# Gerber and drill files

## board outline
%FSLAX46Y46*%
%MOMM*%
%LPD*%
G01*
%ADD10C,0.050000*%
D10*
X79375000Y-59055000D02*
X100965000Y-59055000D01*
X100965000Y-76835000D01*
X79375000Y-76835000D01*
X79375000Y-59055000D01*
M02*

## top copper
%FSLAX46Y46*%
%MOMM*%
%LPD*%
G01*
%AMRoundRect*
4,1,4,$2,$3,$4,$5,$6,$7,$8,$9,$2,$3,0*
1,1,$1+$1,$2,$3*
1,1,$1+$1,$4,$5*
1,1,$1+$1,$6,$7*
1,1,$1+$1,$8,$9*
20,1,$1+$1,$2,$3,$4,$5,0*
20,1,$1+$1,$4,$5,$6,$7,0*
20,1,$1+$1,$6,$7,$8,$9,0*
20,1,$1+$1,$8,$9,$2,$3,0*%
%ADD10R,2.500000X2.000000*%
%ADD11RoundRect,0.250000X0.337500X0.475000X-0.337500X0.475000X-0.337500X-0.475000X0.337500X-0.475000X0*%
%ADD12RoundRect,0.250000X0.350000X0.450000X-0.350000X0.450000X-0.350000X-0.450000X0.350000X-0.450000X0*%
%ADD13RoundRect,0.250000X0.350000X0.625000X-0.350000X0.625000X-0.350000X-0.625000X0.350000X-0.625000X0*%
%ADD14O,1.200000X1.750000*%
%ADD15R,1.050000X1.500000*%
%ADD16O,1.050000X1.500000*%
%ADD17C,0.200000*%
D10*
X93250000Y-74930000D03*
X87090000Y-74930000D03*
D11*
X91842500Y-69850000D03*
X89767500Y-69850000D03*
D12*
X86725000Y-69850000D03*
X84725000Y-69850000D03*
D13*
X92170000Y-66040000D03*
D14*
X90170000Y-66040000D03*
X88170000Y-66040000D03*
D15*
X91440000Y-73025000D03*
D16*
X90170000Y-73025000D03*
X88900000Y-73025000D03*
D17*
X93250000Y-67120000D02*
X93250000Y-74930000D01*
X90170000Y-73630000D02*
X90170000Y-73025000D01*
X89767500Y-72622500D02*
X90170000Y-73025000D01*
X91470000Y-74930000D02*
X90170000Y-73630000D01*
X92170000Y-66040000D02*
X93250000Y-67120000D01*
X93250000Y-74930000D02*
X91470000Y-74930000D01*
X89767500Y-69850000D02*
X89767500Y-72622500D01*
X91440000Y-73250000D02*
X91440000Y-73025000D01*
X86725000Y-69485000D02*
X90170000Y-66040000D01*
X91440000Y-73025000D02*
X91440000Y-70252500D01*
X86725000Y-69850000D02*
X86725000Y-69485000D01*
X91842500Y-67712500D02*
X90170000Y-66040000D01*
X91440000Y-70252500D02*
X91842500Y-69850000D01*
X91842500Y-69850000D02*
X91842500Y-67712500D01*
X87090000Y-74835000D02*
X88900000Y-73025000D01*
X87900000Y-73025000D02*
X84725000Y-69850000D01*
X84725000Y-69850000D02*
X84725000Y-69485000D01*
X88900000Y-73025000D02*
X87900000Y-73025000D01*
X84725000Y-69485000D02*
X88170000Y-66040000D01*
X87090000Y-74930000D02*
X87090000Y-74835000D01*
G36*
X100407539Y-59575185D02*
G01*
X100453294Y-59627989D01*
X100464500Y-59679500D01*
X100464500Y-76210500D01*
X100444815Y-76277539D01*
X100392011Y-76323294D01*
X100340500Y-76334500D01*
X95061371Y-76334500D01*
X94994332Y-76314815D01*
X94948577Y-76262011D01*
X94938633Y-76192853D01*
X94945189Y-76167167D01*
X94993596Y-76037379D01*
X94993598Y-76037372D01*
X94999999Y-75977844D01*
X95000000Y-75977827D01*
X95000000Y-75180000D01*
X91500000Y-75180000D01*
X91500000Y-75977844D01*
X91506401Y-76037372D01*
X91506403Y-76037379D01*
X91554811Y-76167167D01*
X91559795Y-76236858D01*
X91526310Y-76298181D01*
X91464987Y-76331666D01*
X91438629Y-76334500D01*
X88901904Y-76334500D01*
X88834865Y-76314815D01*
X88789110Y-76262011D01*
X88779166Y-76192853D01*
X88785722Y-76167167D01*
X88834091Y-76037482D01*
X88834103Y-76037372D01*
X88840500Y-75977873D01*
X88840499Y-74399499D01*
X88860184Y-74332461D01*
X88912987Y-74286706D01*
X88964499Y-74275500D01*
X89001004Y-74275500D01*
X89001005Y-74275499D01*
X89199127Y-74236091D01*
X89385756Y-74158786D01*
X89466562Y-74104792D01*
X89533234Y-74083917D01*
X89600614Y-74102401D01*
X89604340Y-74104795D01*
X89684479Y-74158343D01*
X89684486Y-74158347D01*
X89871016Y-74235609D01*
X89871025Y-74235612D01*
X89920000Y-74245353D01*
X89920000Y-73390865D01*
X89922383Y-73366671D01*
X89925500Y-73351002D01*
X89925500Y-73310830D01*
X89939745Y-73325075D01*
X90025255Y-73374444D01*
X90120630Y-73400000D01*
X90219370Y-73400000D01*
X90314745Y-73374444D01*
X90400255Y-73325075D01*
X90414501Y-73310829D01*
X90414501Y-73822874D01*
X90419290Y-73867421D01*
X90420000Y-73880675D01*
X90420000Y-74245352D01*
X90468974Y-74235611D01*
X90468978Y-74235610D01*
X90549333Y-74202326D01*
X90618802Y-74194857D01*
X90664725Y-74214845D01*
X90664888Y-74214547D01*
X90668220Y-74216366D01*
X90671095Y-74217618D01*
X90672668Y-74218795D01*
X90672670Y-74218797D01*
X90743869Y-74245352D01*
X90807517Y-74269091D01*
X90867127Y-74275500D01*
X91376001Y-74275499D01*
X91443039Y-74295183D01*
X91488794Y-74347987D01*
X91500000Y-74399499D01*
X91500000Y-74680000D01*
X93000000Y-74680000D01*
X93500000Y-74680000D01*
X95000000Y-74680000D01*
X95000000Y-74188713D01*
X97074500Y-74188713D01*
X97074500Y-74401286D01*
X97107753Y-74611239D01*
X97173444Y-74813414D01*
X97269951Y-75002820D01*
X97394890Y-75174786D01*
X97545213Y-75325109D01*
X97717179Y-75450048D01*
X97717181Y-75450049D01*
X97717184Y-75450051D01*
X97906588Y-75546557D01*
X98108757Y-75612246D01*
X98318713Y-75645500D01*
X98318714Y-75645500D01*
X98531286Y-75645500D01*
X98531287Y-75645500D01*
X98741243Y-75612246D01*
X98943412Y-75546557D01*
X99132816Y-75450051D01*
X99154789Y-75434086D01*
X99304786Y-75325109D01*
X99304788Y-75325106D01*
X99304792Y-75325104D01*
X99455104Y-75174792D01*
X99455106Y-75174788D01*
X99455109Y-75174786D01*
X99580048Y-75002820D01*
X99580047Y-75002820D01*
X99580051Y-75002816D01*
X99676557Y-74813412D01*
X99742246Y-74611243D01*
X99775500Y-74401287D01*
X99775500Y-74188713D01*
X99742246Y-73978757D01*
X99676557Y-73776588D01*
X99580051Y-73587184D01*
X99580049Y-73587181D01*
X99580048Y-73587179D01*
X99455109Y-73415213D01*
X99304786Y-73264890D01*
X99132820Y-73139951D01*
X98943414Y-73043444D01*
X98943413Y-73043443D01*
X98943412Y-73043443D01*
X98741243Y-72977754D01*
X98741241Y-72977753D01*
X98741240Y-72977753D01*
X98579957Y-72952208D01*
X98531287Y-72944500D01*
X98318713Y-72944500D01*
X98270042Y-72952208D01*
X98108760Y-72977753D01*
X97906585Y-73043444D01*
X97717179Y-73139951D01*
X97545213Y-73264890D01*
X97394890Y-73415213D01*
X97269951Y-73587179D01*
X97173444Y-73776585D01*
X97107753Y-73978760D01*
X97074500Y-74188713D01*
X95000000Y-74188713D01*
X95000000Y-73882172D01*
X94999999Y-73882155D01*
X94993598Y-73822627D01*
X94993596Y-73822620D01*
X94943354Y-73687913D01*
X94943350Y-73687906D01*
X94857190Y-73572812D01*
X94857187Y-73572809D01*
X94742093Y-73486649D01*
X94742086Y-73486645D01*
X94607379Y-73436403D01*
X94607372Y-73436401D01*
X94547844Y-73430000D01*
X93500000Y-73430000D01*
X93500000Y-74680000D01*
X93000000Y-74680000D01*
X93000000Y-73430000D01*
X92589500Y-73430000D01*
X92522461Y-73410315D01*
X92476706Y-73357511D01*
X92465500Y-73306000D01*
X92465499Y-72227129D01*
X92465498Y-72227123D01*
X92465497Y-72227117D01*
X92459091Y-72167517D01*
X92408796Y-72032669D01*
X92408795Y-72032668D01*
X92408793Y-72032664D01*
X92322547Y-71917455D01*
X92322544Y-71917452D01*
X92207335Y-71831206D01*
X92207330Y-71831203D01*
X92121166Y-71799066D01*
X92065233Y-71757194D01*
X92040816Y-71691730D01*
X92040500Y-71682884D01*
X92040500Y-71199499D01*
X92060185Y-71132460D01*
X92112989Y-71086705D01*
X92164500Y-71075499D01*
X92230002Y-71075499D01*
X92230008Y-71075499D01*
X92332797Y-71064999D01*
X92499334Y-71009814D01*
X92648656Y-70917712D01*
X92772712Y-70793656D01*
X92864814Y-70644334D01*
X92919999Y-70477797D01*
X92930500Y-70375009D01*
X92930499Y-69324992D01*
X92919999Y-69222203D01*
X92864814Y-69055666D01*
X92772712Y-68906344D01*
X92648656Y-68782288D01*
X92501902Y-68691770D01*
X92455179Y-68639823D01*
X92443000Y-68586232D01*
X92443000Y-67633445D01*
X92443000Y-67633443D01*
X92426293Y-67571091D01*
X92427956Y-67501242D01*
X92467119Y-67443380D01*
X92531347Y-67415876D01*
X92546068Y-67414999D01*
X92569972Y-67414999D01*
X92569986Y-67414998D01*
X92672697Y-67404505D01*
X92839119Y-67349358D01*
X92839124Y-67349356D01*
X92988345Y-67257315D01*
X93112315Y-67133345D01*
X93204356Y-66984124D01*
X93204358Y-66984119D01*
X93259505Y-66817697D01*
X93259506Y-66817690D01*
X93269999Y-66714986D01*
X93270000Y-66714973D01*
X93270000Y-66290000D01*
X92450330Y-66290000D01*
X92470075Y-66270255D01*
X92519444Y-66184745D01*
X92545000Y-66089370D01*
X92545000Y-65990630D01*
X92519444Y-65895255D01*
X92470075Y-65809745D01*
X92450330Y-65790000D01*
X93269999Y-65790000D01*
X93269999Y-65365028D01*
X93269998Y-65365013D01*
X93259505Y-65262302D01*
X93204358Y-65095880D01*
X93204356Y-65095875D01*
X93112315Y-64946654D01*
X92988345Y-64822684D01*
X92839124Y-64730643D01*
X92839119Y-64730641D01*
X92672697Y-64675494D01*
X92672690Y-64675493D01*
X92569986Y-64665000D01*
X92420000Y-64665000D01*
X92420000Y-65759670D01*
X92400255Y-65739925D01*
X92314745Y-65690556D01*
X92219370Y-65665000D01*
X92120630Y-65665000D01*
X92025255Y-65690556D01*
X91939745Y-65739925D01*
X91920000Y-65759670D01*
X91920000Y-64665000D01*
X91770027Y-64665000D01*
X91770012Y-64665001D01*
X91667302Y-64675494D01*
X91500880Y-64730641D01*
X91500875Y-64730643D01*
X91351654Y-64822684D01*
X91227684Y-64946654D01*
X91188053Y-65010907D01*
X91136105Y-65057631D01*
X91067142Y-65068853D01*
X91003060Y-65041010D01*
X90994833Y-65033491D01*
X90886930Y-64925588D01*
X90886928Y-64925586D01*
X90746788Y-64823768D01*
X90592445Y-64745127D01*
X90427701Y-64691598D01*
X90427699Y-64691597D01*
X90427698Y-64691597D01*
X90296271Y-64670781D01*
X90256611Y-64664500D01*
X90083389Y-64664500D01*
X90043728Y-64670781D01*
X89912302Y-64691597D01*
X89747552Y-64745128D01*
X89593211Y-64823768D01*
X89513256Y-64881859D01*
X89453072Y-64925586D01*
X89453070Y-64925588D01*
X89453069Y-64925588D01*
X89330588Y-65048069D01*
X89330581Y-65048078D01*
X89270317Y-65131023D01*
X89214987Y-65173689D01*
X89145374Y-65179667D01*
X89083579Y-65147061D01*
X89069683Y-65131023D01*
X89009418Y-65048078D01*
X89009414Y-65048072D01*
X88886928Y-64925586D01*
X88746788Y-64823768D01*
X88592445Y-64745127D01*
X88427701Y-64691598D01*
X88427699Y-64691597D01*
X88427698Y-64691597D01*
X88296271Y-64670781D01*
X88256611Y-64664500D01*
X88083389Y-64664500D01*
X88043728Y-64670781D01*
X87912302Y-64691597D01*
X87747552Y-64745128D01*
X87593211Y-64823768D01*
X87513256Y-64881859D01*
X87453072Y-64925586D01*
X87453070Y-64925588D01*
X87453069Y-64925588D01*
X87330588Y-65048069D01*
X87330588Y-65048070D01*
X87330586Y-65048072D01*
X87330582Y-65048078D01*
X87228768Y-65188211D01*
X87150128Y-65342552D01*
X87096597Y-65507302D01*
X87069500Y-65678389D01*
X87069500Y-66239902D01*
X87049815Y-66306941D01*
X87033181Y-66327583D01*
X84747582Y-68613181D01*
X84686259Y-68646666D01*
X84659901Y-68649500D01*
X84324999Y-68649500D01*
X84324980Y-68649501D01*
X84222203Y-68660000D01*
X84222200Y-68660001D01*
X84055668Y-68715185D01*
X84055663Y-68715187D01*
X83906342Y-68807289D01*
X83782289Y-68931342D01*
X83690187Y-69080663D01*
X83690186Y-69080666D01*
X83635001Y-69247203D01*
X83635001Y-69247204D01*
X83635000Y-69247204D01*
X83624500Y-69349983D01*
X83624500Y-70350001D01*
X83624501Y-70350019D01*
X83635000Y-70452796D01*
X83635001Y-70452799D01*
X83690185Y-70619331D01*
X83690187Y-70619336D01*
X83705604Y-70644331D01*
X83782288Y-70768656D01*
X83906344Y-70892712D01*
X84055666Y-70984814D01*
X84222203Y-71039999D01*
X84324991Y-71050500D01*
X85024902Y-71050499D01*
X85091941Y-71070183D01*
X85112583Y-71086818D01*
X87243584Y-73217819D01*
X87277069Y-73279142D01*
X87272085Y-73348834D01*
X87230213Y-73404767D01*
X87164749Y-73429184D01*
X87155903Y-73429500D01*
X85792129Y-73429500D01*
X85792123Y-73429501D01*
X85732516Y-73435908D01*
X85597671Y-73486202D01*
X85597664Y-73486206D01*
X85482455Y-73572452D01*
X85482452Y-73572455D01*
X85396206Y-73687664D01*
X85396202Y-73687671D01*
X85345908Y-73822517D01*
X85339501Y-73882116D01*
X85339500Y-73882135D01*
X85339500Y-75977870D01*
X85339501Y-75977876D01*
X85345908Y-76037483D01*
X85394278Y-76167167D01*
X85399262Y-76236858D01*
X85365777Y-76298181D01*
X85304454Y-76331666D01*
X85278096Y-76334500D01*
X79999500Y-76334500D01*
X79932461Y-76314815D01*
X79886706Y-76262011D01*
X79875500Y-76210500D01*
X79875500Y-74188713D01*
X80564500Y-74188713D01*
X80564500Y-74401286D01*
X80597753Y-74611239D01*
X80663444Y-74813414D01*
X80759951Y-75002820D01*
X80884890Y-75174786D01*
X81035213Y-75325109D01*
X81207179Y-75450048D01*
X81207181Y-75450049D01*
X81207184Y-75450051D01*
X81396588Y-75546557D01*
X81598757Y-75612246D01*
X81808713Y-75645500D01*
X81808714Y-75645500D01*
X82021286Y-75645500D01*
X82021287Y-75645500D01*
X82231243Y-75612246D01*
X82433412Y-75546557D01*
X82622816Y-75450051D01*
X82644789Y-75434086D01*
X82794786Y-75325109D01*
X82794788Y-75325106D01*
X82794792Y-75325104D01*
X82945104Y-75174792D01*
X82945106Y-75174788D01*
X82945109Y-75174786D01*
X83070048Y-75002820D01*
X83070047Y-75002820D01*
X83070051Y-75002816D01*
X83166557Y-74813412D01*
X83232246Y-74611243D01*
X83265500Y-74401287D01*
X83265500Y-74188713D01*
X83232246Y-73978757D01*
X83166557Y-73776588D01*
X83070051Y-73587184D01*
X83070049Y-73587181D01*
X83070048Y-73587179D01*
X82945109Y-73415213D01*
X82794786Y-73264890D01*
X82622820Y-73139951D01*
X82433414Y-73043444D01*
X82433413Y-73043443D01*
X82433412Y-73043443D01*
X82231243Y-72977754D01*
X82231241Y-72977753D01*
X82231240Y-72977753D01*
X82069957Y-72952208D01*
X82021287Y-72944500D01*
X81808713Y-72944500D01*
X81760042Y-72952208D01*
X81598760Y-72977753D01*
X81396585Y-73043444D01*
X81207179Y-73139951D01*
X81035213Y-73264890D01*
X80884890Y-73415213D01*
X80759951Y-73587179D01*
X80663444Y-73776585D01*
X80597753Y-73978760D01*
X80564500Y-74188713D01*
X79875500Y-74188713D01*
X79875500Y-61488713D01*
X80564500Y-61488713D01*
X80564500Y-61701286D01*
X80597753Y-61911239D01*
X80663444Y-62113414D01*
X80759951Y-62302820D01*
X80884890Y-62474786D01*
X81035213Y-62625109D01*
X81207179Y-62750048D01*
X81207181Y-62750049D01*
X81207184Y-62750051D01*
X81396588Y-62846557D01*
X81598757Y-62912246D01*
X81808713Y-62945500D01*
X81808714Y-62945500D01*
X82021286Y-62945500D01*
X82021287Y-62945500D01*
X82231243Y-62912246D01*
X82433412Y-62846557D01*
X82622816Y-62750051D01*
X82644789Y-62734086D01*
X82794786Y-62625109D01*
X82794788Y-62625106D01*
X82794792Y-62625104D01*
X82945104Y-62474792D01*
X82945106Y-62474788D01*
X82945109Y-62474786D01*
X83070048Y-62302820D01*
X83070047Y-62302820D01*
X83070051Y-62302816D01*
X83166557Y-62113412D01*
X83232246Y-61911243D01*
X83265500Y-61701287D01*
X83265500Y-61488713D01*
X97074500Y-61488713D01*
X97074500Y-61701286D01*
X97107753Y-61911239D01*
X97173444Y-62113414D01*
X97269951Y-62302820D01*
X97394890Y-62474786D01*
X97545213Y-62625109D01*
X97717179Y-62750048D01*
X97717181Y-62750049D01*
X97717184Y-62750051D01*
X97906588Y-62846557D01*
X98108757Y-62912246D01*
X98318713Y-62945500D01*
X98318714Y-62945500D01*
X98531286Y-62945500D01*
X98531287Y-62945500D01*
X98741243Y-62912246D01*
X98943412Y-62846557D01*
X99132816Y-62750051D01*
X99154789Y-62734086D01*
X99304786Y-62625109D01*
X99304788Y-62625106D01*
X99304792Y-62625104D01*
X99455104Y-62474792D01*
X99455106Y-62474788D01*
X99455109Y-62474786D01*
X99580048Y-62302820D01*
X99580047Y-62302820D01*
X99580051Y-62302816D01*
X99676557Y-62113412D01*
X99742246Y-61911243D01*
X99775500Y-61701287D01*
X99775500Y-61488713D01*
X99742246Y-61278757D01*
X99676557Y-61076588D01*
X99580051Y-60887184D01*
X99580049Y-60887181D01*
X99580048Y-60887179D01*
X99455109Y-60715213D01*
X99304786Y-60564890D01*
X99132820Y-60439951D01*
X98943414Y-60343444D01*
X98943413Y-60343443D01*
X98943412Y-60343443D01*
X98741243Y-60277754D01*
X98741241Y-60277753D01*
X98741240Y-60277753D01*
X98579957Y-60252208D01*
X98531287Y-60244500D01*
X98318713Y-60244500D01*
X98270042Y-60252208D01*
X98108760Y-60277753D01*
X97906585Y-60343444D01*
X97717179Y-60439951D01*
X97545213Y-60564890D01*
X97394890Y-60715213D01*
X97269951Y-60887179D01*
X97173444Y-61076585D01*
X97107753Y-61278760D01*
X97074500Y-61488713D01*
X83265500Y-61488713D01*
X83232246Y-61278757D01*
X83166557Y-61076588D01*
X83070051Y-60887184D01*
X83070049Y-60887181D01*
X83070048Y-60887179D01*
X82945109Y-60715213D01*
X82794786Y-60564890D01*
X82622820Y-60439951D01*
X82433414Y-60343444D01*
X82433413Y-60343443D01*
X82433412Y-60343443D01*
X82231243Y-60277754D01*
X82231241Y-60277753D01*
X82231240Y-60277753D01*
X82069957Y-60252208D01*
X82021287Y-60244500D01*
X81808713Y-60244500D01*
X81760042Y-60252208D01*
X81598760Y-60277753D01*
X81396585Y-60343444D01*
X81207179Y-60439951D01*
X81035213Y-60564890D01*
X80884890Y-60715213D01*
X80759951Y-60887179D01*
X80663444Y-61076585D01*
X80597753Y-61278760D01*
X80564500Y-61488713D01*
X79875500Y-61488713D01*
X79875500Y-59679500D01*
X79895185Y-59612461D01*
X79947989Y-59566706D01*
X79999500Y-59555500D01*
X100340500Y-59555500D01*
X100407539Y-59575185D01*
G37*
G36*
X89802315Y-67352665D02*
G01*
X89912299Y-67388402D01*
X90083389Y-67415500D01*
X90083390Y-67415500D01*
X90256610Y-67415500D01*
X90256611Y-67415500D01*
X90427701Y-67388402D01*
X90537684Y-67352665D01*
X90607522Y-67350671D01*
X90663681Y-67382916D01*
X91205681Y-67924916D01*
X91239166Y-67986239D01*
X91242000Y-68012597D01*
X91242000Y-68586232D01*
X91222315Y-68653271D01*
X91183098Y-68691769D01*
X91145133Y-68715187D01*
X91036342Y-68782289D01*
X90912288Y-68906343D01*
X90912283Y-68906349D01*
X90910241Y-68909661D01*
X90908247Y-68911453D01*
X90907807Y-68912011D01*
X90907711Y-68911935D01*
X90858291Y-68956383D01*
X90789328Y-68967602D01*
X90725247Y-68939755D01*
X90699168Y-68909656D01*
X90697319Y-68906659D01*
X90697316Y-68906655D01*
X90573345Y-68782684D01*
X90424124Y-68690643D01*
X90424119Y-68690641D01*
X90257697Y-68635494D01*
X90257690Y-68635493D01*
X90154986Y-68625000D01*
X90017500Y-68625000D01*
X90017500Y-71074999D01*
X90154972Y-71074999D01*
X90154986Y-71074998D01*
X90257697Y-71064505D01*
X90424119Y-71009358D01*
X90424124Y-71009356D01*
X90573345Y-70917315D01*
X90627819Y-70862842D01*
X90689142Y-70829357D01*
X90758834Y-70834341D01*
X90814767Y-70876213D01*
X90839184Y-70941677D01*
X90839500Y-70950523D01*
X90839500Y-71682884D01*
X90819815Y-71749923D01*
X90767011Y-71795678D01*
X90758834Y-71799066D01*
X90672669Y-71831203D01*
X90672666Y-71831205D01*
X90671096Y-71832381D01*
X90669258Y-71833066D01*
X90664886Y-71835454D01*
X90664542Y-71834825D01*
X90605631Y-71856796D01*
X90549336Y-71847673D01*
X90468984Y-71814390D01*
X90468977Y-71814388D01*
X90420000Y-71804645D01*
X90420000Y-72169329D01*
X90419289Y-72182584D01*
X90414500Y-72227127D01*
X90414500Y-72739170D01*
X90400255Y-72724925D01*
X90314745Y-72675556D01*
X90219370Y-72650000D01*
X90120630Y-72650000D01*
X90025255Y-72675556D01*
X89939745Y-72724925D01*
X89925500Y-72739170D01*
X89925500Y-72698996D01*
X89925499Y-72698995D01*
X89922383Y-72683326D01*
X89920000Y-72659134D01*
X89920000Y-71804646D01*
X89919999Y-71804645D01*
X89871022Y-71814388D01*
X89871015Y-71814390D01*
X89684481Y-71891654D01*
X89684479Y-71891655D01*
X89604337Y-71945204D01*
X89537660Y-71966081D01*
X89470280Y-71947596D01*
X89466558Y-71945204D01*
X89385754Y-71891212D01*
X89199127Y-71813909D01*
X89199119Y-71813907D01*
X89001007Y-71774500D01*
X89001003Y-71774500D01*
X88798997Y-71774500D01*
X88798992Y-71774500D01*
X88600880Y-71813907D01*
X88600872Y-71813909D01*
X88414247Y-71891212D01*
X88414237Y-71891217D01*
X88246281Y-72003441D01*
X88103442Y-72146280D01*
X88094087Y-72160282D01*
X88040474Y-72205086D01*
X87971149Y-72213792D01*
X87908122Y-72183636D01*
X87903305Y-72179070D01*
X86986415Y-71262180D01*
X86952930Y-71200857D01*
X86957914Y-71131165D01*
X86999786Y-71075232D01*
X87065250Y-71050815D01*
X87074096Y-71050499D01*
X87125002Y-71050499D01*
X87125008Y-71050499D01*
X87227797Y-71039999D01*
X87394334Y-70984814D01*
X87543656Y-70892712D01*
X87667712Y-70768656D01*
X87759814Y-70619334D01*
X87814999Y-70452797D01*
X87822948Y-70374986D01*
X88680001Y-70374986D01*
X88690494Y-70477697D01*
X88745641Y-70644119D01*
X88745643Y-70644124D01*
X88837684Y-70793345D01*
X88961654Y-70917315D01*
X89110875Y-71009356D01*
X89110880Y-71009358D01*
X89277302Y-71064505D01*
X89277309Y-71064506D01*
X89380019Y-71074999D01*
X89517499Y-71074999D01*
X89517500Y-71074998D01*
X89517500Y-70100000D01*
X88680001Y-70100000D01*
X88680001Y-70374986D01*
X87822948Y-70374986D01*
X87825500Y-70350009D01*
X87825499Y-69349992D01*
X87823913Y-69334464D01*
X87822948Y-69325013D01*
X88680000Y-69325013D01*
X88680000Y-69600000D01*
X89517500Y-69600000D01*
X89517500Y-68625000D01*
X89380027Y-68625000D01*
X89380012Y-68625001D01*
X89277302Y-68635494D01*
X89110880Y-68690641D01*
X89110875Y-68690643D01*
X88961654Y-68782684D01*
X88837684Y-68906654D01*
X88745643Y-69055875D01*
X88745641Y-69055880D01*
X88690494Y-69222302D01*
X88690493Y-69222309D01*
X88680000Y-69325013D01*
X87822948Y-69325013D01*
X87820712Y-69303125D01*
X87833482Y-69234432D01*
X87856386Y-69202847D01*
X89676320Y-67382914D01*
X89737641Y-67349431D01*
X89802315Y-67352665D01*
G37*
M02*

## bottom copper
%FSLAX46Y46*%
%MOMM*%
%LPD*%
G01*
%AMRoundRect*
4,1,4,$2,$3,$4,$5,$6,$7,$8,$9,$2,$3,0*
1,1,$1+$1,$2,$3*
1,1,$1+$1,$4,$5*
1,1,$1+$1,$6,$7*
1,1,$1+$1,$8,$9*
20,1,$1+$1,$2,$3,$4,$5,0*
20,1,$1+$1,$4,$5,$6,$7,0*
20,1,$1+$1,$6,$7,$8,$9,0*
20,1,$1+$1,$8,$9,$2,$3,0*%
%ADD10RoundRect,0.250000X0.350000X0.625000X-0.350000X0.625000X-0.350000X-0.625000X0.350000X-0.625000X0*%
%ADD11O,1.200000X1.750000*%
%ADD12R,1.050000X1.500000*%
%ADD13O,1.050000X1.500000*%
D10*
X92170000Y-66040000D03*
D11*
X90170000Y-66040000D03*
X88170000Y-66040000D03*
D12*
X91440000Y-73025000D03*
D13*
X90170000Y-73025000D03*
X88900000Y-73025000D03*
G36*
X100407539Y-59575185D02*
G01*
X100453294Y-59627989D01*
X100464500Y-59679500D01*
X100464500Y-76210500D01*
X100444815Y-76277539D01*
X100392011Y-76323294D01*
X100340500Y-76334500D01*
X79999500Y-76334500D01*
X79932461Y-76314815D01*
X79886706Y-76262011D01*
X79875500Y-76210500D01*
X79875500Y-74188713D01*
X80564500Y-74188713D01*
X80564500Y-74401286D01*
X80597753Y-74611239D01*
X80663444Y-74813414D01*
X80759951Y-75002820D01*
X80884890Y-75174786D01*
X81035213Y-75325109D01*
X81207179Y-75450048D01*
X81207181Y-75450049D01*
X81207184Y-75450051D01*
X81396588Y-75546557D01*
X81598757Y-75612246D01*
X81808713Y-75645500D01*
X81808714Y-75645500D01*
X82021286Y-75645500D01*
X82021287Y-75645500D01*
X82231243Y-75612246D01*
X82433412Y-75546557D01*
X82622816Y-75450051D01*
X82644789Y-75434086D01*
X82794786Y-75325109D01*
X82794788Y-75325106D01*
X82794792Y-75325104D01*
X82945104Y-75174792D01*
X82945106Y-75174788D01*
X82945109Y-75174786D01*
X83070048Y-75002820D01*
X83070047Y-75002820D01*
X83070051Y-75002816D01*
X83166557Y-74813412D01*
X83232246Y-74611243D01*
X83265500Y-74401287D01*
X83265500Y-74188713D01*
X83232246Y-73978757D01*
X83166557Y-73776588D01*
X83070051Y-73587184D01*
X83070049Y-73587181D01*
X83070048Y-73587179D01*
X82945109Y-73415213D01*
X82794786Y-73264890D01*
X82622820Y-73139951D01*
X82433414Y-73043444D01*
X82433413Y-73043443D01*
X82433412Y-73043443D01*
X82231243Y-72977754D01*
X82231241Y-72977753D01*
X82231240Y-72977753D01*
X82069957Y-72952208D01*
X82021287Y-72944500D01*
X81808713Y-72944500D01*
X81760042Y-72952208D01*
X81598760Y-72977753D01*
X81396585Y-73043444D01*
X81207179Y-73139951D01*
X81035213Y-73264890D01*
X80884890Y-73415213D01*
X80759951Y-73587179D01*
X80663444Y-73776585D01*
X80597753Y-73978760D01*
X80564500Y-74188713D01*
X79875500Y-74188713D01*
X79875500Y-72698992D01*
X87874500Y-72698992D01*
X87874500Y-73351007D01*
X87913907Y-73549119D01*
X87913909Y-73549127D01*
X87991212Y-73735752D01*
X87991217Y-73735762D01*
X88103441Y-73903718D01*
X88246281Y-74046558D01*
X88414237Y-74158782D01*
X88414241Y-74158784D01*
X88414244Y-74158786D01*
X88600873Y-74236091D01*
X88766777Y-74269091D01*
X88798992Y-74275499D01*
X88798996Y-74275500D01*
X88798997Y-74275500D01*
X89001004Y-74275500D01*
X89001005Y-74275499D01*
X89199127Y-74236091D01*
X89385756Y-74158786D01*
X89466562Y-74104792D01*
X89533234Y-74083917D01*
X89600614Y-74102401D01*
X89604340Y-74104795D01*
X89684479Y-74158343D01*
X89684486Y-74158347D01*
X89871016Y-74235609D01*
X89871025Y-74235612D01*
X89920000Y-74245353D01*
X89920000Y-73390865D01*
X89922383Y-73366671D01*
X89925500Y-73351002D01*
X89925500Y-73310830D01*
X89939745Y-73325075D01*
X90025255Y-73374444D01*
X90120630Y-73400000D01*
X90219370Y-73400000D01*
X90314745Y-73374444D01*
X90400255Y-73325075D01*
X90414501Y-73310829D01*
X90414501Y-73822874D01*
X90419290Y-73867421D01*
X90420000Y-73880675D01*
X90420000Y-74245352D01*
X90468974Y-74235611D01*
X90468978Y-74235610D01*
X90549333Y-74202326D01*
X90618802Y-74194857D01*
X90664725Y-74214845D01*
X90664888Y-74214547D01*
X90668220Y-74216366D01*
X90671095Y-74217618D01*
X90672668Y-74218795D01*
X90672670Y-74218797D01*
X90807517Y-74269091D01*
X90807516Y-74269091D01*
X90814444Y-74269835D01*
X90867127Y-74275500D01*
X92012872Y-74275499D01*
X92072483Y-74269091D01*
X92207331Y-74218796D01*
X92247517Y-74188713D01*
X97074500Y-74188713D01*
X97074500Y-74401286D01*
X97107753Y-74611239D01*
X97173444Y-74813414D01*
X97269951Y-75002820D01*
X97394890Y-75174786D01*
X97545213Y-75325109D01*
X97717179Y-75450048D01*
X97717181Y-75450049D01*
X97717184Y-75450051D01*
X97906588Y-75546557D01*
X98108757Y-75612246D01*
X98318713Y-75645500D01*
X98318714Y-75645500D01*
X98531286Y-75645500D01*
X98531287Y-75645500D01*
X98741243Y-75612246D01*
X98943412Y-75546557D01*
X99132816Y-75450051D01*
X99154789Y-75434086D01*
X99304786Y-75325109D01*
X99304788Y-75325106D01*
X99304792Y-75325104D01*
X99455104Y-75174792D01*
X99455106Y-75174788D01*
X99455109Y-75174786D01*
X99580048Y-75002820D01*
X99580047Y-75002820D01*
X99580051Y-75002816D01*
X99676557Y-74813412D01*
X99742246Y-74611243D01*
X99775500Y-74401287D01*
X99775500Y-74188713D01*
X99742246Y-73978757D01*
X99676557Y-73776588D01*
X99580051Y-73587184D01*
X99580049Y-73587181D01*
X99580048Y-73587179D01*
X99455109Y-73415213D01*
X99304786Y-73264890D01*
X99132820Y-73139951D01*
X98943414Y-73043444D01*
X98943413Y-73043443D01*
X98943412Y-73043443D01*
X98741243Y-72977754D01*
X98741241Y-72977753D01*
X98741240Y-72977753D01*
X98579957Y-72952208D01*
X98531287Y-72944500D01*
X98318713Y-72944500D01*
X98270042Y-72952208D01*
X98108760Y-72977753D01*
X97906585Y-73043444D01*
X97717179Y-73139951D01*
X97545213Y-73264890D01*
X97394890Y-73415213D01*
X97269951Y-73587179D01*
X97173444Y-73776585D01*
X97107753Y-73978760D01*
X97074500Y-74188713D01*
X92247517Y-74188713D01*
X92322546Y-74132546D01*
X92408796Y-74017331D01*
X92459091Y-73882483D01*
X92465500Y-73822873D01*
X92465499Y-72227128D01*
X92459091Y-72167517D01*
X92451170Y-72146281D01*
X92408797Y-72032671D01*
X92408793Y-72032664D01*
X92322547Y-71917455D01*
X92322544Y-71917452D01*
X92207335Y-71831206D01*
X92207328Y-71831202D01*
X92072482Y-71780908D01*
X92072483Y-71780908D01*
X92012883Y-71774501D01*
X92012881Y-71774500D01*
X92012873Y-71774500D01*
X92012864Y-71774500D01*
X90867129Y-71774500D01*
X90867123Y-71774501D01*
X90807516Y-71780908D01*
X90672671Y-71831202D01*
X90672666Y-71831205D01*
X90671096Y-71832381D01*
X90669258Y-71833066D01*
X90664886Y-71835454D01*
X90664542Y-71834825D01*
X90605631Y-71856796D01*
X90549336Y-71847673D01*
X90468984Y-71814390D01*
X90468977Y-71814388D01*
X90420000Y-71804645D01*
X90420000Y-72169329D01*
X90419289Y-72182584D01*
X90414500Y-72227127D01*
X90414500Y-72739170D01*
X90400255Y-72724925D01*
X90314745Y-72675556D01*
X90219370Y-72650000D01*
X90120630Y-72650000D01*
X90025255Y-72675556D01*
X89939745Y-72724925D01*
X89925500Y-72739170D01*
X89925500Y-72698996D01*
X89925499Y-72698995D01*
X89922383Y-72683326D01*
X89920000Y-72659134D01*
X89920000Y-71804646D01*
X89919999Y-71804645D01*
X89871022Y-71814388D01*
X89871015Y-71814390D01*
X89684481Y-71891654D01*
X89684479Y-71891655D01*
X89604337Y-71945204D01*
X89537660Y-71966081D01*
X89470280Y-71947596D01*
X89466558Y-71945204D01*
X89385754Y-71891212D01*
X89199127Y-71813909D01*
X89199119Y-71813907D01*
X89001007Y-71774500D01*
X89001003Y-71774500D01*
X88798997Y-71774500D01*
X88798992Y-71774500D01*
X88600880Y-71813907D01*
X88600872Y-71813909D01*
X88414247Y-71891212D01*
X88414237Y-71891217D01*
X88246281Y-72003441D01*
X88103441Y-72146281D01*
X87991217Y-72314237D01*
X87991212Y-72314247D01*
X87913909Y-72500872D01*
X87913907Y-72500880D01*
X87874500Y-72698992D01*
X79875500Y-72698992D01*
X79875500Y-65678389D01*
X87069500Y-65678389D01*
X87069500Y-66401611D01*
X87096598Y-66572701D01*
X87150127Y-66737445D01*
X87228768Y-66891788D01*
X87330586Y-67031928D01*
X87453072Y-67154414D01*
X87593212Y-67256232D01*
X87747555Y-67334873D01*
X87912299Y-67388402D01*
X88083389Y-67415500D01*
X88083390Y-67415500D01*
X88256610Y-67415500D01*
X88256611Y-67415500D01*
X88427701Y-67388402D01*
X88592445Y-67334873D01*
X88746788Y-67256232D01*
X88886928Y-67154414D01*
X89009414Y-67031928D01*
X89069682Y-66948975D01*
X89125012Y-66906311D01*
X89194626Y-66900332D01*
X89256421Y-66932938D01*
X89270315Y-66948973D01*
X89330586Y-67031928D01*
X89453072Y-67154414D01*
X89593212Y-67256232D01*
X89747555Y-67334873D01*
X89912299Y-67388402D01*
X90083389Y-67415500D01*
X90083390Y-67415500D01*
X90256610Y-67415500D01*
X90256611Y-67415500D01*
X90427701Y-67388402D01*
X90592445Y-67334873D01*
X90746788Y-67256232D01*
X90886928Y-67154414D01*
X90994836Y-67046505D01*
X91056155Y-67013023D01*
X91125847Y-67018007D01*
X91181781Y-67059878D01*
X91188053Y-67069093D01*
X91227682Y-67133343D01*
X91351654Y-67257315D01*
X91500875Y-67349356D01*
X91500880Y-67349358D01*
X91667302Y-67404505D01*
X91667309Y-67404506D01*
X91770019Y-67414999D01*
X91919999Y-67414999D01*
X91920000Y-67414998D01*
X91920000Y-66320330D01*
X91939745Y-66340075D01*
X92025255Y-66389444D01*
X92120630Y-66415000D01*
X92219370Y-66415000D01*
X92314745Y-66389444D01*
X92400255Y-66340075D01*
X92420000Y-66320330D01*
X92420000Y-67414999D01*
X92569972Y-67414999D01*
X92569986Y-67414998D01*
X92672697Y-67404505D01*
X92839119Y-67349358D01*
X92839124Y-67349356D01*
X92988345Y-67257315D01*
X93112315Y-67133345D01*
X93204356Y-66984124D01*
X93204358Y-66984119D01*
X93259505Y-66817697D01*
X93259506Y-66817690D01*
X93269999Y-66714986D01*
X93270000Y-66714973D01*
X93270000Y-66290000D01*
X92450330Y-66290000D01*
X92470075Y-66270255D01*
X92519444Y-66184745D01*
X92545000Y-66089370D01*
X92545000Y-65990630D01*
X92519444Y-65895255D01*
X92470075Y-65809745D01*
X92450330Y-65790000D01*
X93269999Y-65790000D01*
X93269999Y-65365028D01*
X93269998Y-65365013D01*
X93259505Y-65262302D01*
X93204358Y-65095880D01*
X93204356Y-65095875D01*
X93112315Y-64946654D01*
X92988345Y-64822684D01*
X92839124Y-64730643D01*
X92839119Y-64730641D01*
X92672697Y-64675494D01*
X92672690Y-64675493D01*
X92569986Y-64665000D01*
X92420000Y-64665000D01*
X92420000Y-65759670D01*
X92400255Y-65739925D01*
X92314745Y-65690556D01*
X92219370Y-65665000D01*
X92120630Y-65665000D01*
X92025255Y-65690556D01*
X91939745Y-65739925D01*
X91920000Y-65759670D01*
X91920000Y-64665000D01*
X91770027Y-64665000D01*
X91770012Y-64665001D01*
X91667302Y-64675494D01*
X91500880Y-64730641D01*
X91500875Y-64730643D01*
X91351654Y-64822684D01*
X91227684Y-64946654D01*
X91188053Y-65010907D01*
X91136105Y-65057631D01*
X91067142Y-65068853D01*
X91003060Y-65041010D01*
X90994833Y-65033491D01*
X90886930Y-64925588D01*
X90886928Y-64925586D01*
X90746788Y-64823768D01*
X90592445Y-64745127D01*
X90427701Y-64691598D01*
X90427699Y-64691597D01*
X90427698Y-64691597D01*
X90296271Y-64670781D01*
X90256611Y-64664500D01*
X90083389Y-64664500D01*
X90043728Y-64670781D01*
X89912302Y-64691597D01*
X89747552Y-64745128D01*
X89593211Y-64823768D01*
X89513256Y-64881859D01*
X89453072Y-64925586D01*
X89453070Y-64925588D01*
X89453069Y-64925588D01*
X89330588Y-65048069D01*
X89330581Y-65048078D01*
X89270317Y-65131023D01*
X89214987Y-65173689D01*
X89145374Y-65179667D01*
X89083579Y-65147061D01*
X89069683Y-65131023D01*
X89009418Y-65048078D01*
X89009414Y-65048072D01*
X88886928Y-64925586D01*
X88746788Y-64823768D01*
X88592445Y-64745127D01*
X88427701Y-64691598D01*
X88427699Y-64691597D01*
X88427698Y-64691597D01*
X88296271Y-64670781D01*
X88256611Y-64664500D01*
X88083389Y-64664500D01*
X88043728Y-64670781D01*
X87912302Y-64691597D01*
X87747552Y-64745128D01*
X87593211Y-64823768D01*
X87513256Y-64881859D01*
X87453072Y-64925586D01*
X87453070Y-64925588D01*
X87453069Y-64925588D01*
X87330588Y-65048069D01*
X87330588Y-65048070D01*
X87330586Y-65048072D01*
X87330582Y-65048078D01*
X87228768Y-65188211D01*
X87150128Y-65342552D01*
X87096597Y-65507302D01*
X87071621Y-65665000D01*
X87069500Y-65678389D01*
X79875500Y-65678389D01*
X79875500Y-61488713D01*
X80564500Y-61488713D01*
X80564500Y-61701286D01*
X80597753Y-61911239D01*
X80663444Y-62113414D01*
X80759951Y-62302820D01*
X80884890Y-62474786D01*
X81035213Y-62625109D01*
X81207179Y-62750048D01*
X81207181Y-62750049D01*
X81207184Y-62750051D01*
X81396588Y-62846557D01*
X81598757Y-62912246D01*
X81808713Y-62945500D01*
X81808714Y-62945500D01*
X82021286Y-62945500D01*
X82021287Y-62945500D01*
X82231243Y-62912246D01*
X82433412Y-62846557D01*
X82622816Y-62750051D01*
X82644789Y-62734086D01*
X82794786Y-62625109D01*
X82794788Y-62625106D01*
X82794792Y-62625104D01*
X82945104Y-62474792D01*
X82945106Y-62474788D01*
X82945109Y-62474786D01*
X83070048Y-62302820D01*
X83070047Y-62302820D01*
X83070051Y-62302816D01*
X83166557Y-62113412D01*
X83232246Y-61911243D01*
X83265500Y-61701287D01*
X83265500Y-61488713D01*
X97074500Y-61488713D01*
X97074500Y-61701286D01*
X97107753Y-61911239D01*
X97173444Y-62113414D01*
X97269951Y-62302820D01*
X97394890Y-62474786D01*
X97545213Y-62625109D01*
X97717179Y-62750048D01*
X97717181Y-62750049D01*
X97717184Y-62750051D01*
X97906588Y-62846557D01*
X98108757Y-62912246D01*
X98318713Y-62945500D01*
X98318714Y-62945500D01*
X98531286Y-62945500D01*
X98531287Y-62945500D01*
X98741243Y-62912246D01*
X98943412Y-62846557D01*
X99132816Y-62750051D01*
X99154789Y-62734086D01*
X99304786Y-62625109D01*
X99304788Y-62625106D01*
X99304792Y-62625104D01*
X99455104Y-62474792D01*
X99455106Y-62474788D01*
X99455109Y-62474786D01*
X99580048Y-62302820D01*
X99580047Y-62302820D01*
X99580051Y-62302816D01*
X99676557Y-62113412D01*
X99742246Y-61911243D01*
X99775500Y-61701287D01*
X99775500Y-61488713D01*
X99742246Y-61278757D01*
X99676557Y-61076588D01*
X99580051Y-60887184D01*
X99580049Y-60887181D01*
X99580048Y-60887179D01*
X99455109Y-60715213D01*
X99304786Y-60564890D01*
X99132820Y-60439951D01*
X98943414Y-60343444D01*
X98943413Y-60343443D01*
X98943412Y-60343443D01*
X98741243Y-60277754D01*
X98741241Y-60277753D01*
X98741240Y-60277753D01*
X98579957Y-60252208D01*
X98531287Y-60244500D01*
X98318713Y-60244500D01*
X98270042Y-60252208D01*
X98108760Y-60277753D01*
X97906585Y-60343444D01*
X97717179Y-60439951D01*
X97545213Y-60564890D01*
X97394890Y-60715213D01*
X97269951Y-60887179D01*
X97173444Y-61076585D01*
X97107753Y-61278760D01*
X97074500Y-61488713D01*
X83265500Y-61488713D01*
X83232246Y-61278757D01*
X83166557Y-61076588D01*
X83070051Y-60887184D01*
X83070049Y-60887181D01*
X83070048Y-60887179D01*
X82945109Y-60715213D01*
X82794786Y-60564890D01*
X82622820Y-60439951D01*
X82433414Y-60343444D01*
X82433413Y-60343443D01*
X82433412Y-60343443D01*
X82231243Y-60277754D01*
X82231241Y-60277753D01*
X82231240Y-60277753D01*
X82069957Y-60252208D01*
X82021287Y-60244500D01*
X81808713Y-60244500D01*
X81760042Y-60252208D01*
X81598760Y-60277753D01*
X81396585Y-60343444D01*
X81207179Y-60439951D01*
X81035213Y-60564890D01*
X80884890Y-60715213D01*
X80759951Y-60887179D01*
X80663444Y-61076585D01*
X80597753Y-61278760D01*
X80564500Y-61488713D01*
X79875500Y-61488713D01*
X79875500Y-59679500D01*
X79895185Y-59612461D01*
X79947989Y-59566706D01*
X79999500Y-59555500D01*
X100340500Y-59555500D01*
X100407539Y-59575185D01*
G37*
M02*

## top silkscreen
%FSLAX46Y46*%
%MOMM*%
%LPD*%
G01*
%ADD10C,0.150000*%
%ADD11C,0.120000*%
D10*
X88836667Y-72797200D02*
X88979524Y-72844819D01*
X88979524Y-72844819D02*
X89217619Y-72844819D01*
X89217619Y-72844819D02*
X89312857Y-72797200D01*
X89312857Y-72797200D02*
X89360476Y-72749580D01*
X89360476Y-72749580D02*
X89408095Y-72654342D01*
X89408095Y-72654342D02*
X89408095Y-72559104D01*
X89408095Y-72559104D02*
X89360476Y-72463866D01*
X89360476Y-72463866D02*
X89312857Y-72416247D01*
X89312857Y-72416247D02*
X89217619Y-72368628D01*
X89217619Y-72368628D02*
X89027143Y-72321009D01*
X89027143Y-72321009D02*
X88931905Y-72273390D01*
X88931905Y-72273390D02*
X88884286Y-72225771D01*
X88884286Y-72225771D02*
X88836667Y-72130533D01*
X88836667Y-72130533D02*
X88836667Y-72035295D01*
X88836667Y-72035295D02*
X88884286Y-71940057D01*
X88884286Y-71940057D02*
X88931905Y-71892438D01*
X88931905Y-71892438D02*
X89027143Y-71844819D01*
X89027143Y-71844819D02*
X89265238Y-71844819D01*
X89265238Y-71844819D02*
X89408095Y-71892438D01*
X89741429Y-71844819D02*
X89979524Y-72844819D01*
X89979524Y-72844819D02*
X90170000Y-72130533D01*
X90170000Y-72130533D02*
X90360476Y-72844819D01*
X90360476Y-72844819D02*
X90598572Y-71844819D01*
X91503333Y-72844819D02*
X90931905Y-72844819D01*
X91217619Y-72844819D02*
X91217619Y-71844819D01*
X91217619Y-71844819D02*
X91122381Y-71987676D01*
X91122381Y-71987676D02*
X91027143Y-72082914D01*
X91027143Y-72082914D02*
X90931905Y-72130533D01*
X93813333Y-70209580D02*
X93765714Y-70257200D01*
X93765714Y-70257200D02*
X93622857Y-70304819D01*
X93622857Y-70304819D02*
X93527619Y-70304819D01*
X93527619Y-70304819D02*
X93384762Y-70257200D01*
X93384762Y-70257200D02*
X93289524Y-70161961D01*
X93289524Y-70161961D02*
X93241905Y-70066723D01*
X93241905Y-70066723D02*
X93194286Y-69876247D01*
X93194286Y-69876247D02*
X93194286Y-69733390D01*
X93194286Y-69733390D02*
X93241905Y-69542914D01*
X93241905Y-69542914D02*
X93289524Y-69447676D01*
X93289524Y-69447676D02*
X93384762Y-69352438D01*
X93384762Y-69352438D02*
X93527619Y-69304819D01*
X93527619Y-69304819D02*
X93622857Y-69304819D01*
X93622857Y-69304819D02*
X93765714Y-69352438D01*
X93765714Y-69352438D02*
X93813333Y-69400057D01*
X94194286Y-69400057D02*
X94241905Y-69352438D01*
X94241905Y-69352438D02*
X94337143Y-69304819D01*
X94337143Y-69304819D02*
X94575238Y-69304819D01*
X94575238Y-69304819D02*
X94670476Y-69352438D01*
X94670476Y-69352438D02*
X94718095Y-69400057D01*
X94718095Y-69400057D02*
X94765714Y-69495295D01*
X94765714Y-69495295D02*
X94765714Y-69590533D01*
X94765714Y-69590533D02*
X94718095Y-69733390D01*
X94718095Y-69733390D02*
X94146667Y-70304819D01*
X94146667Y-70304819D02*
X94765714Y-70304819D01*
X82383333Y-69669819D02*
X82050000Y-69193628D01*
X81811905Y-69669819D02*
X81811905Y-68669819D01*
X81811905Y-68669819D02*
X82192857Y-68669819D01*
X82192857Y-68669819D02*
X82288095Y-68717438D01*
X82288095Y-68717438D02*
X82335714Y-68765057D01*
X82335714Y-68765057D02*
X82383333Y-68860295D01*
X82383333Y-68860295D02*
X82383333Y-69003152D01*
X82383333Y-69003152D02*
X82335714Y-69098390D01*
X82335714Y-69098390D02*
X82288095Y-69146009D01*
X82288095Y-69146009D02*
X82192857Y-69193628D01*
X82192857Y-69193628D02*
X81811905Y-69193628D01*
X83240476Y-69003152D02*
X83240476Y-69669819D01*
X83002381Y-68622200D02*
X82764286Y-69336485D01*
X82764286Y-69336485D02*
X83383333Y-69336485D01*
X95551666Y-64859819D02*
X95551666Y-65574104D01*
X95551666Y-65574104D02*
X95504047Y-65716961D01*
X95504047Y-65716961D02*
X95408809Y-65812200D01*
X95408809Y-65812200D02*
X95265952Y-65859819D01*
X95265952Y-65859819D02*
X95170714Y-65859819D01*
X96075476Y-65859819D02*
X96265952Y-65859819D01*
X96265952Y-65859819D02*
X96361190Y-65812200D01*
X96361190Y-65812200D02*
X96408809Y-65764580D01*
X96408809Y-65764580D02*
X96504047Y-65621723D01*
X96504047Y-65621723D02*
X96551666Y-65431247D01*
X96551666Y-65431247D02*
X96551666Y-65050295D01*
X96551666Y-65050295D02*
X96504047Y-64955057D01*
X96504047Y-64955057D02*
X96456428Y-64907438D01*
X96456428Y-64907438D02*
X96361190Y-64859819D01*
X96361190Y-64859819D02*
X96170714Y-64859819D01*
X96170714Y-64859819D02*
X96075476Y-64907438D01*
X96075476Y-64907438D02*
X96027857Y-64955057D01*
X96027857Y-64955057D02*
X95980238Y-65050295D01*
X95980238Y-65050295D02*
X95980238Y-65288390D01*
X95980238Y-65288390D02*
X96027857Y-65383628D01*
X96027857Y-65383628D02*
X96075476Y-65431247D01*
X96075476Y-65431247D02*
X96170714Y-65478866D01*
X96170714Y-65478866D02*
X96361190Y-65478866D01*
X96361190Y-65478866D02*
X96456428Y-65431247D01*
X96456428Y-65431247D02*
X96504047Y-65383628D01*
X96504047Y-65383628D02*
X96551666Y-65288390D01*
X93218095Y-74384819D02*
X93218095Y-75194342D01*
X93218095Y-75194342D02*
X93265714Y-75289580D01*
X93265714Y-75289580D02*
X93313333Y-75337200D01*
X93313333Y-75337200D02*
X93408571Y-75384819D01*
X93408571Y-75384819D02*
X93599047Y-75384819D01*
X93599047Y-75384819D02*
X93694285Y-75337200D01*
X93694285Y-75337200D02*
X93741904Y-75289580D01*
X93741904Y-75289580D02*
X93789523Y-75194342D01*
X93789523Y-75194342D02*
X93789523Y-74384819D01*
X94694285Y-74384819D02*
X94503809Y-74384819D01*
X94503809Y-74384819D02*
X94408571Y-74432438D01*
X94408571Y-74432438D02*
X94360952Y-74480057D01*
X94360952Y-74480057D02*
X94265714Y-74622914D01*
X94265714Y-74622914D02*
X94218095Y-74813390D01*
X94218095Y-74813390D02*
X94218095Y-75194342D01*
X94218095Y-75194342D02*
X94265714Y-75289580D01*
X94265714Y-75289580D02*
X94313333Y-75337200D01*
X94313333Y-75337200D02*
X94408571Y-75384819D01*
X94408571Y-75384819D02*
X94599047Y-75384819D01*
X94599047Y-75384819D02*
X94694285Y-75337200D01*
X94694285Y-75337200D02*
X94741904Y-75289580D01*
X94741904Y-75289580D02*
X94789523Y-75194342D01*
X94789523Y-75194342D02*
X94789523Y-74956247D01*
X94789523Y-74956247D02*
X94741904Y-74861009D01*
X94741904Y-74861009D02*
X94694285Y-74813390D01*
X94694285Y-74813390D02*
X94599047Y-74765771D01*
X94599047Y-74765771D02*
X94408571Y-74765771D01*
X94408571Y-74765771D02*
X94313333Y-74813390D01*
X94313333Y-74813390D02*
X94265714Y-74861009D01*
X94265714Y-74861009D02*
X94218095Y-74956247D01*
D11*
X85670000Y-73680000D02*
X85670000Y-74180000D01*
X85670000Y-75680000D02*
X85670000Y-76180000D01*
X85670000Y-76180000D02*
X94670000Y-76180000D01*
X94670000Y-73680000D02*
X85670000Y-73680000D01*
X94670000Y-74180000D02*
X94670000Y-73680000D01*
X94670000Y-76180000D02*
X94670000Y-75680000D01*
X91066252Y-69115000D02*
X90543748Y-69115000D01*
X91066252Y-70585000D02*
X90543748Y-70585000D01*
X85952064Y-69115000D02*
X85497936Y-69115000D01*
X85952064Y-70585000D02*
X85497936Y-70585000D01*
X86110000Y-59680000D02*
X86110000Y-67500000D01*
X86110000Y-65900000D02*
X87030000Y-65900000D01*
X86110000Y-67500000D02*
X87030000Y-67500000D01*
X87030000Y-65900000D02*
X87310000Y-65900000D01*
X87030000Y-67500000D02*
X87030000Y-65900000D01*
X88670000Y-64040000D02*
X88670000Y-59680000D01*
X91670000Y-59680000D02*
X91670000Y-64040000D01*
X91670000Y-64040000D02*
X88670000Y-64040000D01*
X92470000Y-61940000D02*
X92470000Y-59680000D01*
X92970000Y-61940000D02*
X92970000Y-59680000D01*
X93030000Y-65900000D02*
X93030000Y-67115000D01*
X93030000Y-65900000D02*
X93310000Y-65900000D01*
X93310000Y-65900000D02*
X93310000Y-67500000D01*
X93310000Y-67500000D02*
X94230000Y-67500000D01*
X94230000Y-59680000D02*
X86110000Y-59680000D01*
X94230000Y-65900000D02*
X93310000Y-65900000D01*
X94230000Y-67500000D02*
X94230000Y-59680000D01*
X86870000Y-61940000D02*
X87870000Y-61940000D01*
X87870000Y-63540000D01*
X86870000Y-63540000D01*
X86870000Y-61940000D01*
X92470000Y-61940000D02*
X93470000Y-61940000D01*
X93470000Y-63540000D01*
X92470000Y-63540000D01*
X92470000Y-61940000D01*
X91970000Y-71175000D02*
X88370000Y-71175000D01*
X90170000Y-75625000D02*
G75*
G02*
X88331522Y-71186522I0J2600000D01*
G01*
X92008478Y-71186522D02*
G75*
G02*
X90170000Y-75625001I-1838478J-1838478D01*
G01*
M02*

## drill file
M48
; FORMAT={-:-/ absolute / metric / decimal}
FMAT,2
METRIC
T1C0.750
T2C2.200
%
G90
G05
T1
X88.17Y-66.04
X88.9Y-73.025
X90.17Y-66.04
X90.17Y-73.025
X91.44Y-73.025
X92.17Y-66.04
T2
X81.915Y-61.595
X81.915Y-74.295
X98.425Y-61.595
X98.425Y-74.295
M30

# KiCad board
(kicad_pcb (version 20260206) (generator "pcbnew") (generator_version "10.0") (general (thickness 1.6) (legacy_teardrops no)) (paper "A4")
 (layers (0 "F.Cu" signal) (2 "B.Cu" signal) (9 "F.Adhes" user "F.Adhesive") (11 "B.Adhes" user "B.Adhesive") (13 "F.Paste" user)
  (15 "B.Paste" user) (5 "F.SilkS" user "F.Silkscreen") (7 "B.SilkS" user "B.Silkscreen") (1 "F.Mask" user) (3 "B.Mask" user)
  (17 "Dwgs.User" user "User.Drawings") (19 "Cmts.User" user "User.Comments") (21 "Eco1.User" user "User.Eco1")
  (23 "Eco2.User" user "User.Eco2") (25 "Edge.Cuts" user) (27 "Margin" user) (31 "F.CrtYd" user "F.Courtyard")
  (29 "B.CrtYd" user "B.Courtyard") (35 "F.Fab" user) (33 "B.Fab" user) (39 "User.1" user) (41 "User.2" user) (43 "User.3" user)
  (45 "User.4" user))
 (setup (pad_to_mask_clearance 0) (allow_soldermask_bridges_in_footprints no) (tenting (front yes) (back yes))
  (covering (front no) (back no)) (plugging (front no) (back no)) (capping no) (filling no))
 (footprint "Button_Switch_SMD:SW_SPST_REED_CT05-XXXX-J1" (layer "F.Cu") (at 90.17 74.93 180)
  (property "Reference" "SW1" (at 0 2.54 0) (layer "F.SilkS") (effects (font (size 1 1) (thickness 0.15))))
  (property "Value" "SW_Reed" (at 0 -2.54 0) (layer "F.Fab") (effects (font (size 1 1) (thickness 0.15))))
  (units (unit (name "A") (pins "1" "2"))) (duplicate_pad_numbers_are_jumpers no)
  (fp_line (start 4.5 1.25) (end 4.5 0.75) (stroke (width 0.12) (type solid)) (layer "F.SilkS"))
  (fp_line (start 4.5 -0.75) (end 4.5 -1.25) (stroke (width 0.12) (type solid)) (layer "F.SilkS"))
  (fp_line (start 4.5 -1.25) (end -4.5 -1.25) (stroke (width 0.12) (type solid)) (layer "F.SilkS"))
  (fp_line (start -4.5 1.25) (end 4.5 1.25) (stroke (width 0.12) (type solid)) (layer "F.SilkS"))
  (fp_line (start -4.5 0.75) (end -4.5 1.25) (stroke (width 0.12) (type solid)) (layer "F.SilkS"))
  (fp_line (start -4.5 -1.25) (end -4.5 -0.75) (stroke (width 0.12) (type solid)) (layer "F.SilkS"))
  (pad "1" smd rect (at -3.08 0 180) (size 2.5 2) (layers "F.Cu" "F.Mask" "F.Paste") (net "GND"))
  (pad "2" smd rect (at 3.08 0 180) (size 2.5 2) (layers "F.Cu" "F.Mask" "F.Paste") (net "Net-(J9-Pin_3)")))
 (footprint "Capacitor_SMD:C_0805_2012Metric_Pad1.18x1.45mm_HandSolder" (layer "F.Cu") (at 90.805 69.85 180)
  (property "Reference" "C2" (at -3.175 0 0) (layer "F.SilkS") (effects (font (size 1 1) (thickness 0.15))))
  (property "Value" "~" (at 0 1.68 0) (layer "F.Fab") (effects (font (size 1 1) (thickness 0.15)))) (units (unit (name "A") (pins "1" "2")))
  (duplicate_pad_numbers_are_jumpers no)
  (fp_line (start -0.261252 0.735) (end 0.261252 0.735) (stroke (width 0.12) (type solid)) (layer "F.SilkS"))
  (fp_line (start -0.261252 -0.735) (end 0.261252 -0.735) (stroke (width 0.12) (type solid)) (layer "F.SilkS"))
  (pad "1" smd roundrect (at -1.0375 0 180) (size 1.175 1.45) (layers "F.Cu" "F.Mask" "F.Paste") (roundrect_rratio 0.212766) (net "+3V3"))
  (pad "2" smd roundrect (at 1.0375 0 180) (size 1.175 1.45) (layers "F.Cu" "F.Mask" "F.Paste") (roundrect_rratio 0.212766) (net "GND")))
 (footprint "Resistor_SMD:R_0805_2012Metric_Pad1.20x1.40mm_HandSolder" (layer "F.Cu") (at 85.725 69.85 180)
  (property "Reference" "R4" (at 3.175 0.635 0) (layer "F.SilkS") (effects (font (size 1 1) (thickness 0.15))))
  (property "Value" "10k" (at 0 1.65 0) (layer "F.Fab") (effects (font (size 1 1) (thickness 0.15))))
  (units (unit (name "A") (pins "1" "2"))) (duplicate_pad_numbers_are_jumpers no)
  (fp_line (start -0.227064 0.735) (end 0.227064 0.735) (stroke (width 0.12) (type solid)) (layer "F.SilkS"))
  (fp_line (start -0.227064 -0.735) (end 0.227064 -0.735) (stroke (width 0.12) (type solid)) (layer "F.SilkS"))
  (pad "1" smd roundrect (at -1 0 180) (size 1.2 1.4) (layers "F.Cu" "F.Mask" "F.Paste") (roundrect_rratio 0.208333) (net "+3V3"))
  (pad "2" smd roundrect (at 1 0 180) (size 1.2 1.4) (layers "F.Cu" "F.Mask" "F.Paste") (roundrect_rratio 0.208333) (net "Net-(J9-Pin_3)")))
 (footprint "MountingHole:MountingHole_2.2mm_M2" (layer "F.Cu") (at 98.425 61.595)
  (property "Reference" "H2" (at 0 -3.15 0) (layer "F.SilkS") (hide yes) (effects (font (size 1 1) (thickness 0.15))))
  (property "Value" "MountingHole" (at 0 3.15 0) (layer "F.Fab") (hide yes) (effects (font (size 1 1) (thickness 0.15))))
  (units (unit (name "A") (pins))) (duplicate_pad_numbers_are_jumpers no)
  (pad "" np_thru_hole circle (at 0 0) (size 2.2 2.2) (drill 2.2) (layers "*.Cu" "*.Mask")))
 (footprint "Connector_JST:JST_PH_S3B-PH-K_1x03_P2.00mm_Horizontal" (layer "F.Cu") (at 92.17 66.04 180)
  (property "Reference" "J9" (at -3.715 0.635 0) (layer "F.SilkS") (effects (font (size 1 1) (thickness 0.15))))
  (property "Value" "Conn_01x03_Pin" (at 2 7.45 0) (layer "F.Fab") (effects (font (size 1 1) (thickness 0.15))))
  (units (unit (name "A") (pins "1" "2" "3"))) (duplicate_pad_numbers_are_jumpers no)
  (fp_line (start 6.06 6.36) (end 6.06 -1.46) (stroke (width 0.12) (type solid)) (layer "F.SilkS"))
  (fp_line (start 6.06 0.14) (end 5.14 0.14) (stroke (width 0.12) (type solid)) (layer "F.SilkS"))
  (fp_line (start 6.06 -1.46) (end 5.14 -1.46) (stroke (width 0.12) (type solid)) (layer "F.SilkS"))
  (fp_line (start 5.14 0.14) (end 4.86 0.14) (stroke (width 0.12) (type solid)) (layer "F.SilkS"))
  (fp_line (start 5.14 -1.46) (end 5.14 0.14) (stroke (width 0.12) (type solid)) (layer "F.SilkS"))
  (fp_line (start 3.5 2) (end 3.5 6.36) (stroke (width 0.12) (type solid)) (layer "F.SilkS"))
  (fp_line (start 0.5 6.36) (end 0.5 2) (stroke (width 0.12) (type solid)) (layer "F.SilkS"))
  (fp_line (start 0.5 2) (end 3.5 2) (stroke (width 0.12) (type solid)) (layer "F.SilkS"))
  (fp_line (start -0.3 4.1) (end -0.3 6.36) (stroke (width 0.12) (type solid)) (layer "F.SilkS"))
  (fp_line (start -0.8 4.1) (end -0.8 6.36) (stroke (width 0.12) (type solid)) (layer "F.SilkS"))
  (fp_line (start -0.86 0.14) (end -0.86 -1.075) (stroke (width 0.12) (type solid)) (layer "F.SilkS"))
  (fp_line (start -0.86 0.14) (end -1.14 0.14) (stroke (width 0.12) (type solid)) (layer "F.SilkS"))
  (fp_line (start -1.14 0.14) (end -1.14 -1.46) (stroke (width 0.12) (type solid)) (layer "F.SilkS"))
  (fp_line (start -1.14 -1.46) (end -2.06 -1.46) (stroke (width 0.12) (type solid)) (layer "F.SilkS"))
  (fp_line (start -2.06 6.36) (end 6.06 6.36) (stroke (width 0.12) (type solid)) (layer "F.SilkS"))
  (fp_line (start -2.06 0.14) (end -1.14 0.14) (stroke (width 0.12) (type solid)) (layer "F.SilkS"))
  (fp_line (start -2.06 -1.46) (end -2.06 6.36) (stroke (width 0.12) (type solid)) (layer "F.SilkS"))
  (fp_rect (start 4.3 2.5) (end 5.3 4.1) (stroke (width 0.12) (type solid)) (fill no) (layer "F.SilkS"))
  (fp_rect (start -1.3 2.5) (end -0.3 4.1) (stroke (width 0.12) (type solid)) (fill no) (layer "F.SilkS"))
  (pad "1" thru_hole roundrect (at 0 0 180) (size 1.2 1.75) (drill 0.75) (layers "*.Cu" "*.Mask") (remove_unused_layers no)
   (roundrect_rratio 0.208333) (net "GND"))
  (pad "2" thru_hole oval (at 2 0 180) (size 1.2 1.75) (drill 0.75) (layers "*.Cu" "*.Mask") (remove_unused_layers no) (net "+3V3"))
  (pad "3" thru_hole oval (at 4 0 180) (size 1.2 1.75) (drill 0.75) (layers "*.Cu" "*.Mask") (remove_unused_layers no)
   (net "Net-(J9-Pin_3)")))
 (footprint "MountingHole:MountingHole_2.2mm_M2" (layer "F.Cu") (at 81.915 74.295)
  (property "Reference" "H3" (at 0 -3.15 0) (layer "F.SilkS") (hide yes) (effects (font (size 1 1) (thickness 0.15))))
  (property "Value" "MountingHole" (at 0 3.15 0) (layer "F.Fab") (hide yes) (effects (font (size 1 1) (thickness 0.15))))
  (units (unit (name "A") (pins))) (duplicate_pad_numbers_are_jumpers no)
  (pad "" np_thru_hole circle (at 0 0) (size 2.2 2.2) (drill 2.2) (layers "*.Cu" "*.Mask")))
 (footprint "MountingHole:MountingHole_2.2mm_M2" (layer "F.Cu") (at 98.425 74.295)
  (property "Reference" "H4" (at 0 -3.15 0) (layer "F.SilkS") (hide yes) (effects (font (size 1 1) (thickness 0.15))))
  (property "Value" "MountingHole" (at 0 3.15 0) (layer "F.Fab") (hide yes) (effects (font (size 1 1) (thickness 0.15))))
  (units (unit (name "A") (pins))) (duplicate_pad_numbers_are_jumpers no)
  (pad "" np_thru_hole circle (at 0 0) (size 2.2 2.2) (drill 2.2) (layers "*.Cu" "*.Mask")))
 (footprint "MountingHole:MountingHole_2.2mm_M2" (layer "F.Cu") (at 81.915 61.595)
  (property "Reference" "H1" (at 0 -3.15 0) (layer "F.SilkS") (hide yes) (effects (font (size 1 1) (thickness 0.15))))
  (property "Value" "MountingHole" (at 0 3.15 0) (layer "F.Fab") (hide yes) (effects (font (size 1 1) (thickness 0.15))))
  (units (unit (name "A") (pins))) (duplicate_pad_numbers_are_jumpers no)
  (pad "" np_thru_hole circle (at 0 0) (size 2.2 2.2) (drill 2.2) (layers "*.Cu" "*.Mask")))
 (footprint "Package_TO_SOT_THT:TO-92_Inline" (layer "F.Cu") (at 91.44 73.025 180)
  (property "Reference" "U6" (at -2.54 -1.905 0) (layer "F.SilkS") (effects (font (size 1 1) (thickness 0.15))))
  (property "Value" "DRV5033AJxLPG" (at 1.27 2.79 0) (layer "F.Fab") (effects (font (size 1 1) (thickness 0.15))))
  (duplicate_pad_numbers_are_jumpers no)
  (fp_line (start -0.53 1.85) (end 3.07 1.85) (stroke (width 0.12) (type solid)) (layer "F.SilkS"))
  (fp_arc (start 1.27 -2.6) (mid 3.672087 -0.994977) (end 3.108478 1.838478) (stroke (width 0.12) (type solid)) (layer "F.SilkS"))
  (fp_arc (start -0.568478 1.838478) (mid -1.132087 -0.994977) (end 1.27 -2.6) (stroke (width 0.12) (type solid)) (layer "F.SilkS"))
  (pad "1" thru_hole rect (at 0 0 180) (size 1.05 1.5) (drill 0.75) (layers "*.Cu" "*.Mask") (remove_unused_layers no) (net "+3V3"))
  (pad "2" thru_hole oval (at 1.27 0 180) (size 1.05 1.5) (drill 0.75) (layers "*.Cu" "*.Mask") (remove_unused_layers no) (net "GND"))
  (pad "3" thru_hole oval (at 2.54 0 180) (size 1.05 1.5) (drill 0.75) (layers "*.Cu" "*.Mask") (remove_unused_layers no)
   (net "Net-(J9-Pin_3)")))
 (gr_rect (start 79.375 59.055) (end 100.965 76.835) (stroke (width 0.05) (type solid)) (fill no) (layer "Edge.Cuts"))
 (segment (start 93.25 67.12) (end 93.25 74.93) (width 0.2) (layer "F.Cu") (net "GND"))
 (segment (start 90.17 73.63) (end 90.17 73.025) (width 0.2) (layer "F.Cu") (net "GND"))
 (segment (start 89.7675 72.6225) (end 90.17 73.025) (width 0.2) (layer "F.Cu") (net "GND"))
 (segment (start 91.47 74.93) (end 90.17 73.63) (width 0.2) (layer "F.Cu") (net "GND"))
 (segment (start 92.17 66.04) (end 93.25 67.12) (width 0.2) (layer "F.Cu") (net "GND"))
 (segment (start 93.25 74.93) (end 91.47 74.93) (width 0.2) (layer "F.Cu") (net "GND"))
 (segment (start 89.7675 69.85) (end 89.7675 72.6225) (width 0.2) (layer "F.Cu") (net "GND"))
 (segment (start 91.44 73.25) (end 91.44 73.025) (width 0.2) (layer "F.Cu") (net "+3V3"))
 (segment (start 86.725 69.485) (end 90.17 66.04) (width 0.2) (layer "F.Cu") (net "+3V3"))
 (segment (start 91.44 73.025) (end 91.44 70.2525) (width 0.2) (layer "F.Cu") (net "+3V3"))
 (segment (start 86.725 69.85) (end 86.725 69.485) (width 0.2) (layer "F.Cu") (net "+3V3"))
 (segment (start 91.8425 67.7125) (end 90.17 66.04) (width 0.2) (layer "F.Cu") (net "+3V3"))
 (segment (start 91.44 70.2525) (end 91.8425 69.85) (width 0.2) (layer "F.Cu") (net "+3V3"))
 (segment (start 91.8425 69.85) (end 91.8425 67.7125) (width 0.2) (layer "F.Cu") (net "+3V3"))
 (segment (start 87.09 74.835) (end 88.9 73.025) (width 0.2) (layer "F.Cu") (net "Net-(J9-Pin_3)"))
 (segment (start 87.9 73.025) (end 84.725 69.85) (width 0.2) (layer "F.Cu") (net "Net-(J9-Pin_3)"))
 (segment (start 84.725 69.85) (end 84.725 69.485) (width 0.2) (layer "F.Cu") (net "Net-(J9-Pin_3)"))
 (segment (start 88.9 73.025) (end 87.9 73.025) (width 0.2) (layer "F.Cu") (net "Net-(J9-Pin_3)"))
 (segment (start 84.725 69.485) (end 88.17 66.04) (width 0.2) (layer "F.Cu") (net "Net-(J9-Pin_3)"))
 (segment (start 87.09 74.93) (end 87.09 74.835) (width 0.2) (layer "F.Cu") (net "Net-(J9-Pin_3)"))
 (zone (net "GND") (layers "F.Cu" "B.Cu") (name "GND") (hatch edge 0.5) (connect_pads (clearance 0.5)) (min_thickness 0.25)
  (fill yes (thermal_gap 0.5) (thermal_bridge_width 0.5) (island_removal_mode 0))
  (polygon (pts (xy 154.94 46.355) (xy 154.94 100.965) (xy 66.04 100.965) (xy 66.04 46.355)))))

